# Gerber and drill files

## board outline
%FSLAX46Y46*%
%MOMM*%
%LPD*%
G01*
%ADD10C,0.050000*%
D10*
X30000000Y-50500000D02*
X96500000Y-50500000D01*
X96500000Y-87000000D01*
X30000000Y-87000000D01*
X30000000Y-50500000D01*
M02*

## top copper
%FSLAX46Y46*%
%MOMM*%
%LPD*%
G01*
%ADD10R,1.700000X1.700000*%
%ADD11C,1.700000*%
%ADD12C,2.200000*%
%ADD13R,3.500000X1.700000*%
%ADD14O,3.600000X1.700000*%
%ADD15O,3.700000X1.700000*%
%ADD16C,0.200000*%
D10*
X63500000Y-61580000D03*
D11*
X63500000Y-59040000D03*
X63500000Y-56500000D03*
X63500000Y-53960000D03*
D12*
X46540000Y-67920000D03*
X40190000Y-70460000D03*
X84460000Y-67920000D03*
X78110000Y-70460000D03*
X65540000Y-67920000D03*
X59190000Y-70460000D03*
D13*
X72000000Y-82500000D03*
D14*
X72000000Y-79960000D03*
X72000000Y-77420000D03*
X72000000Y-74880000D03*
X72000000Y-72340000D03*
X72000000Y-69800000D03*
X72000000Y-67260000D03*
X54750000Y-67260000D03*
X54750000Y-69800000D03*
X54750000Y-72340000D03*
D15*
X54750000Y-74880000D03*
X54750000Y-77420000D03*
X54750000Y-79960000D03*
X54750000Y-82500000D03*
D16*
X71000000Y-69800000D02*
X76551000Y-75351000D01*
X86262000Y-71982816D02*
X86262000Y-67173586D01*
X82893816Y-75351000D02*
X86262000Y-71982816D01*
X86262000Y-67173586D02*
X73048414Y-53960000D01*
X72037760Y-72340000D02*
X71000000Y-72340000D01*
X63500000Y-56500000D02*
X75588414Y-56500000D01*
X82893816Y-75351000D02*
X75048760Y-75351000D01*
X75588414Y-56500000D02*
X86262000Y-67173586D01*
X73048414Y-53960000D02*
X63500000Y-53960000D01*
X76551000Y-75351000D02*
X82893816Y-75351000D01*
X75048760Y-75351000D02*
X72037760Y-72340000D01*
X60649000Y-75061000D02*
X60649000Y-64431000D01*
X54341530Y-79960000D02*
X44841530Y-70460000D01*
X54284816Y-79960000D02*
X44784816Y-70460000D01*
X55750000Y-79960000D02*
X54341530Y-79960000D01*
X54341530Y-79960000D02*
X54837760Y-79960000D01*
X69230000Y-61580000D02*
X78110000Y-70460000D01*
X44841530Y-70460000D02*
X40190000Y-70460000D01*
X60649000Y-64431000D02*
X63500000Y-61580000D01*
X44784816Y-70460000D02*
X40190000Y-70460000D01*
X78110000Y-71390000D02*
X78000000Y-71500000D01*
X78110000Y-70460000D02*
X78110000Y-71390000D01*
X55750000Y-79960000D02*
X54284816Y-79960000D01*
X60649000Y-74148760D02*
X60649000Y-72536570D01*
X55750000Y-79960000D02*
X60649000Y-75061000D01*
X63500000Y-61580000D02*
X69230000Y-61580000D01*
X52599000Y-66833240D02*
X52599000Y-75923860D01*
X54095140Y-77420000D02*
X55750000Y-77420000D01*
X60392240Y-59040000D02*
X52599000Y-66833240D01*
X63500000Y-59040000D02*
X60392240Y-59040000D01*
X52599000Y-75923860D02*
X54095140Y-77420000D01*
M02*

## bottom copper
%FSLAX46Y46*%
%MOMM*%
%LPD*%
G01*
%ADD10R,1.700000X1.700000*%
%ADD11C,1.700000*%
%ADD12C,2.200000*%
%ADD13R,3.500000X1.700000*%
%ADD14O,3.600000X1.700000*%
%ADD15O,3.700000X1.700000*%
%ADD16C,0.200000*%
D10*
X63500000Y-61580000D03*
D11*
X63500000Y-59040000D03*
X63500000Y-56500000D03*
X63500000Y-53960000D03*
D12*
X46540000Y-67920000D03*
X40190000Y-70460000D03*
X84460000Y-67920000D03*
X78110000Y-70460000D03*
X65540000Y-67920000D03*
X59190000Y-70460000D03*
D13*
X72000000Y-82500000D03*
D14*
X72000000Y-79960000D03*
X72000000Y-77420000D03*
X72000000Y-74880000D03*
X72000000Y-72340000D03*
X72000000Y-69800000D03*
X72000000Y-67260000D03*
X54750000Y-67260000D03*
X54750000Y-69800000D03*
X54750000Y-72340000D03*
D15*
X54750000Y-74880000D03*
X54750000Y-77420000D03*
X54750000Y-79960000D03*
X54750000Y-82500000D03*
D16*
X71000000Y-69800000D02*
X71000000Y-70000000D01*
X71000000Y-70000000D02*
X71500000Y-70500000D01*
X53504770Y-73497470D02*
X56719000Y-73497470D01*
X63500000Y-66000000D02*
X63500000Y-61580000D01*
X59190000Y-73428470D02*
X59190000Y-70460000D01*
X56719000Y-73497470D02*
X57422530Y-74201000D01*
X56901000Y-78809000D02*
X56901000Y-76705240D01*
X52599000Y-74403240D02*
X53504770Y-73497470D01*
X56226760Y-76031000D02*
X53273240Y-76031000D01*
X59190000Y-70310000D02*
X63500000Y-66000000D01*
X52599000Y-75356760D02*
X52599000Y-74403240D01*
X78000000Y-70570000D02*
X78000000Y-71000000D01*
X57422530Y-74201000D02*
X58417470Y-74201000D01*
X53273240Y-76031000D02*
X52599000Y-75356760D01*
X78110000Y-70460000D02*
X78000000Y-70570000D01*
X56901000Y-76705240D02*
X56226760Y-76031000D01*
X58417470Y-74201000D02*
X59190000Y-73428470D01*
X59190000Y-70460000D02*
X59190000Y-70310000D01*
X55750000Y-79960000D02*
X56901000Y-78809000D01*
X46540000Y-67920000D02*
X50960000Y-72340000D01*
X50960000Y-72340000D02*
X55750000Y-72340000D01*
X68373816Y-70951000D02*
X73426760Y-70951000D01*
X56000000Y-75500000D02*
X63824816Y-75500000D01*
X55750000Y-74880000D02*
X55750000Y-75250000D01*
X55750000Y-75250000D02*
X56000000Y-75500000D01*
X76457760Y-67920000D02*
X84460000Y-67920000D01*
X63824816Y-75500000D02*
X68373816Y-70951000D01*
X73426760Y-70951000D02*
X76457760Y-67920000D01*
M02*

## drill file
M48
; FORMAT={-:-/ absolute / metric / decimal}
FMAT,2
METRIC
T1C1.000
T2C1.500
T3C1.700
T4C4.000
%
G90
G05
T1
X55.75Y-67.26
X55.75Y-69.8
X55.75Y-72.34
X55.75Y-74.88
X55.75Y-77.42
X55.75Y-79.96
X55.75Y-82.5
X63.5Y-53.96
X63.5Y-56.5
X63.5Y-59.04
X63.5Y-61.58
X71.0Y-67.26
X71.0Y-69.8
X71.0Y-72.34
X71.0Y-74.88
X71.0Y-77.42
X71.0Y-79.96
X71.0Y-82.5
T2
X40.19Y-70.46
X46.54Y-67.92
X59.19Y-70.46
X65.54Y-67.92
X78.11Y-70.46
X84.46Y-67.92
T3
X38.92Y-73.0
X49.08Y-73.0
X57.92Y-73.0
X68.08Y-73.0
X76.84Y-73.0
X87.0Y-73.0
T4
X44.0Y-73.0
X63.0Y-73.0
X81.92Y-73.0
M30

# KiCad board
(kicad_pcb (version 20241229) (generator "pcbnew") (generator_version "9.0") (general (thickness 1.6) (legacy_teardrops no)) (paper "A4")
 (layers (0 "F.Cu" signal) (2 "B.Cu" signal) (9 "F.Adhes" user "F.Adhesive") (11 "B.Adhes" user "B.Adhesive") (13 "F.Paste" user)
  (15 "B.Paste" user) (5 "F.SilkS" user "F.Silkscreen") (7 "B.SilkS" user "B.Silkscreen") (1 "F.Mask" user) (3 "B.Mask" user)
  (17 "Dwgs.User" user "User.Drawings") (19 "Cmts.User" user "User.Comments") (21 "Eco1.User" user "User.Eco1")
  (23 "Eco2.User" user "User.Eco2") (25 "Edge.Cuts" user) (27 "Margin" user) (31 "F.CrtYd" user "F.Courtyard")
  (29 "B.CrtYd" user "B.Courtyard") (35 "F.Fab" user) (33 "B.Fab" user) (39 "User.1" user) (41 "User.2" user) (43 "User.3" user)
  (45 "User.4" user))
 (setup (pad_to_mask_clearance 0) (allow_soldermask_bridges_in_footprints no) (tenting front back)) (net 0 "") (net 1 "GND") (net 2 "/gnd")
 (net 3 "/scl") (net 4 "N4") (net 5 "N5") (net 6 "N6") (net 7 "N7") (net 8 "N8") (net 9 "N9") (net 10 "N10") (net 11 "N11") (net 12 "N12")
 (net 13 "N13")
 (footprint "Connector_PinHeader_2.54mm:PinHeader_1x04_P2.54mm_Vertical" (layer "F.Cu") (at 63.5 61.58 180)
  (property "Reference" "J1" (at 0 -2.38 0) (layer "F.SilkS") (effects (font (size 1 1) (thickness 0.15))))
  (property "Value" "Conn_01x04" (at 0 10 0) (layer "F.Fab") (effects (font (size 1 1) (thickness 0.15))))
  (pad "1" thru_hole rect (at 0 0 180) (size 1.7 1.7) (drill 1) (layers "*.Cu" "*.Mask") (remove_unused_layers no) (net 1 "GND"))
  (pad "2" thru_hole circle (at 0 2.54 180) (size 1.7 1.7) (drill 1) (layers "*.Cu" "*.Mask") (remove_unused_layers no) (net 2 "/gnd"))
  (pad "3" thru_hole circle (at 0 5.08 180) (size 1.7 1.7) (drill 1) (layers "*.Cu" "*.Mask") (remove_unused_layers no) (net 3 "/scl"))
  (pad "4" thru_hole circle (at 0 7.62 180) (size 1.7 1.7) (drill 1) (layers "*.Cu" "*.Mask") (remove_unused_layers no) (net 3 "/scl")))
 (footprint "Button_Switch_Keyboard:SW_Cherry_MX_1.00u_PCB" (layer "F.Cu") (at 46.54 67.92)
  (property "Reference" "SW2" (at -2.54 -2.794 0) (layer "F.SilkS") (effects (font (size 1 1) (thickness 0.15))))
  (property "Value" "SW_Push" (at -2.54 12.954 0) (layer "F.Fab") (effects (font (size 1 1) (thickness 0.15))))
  (pad "" np_thru_hole circle (at -7.62 5.08) (size 1.7 1.7) (drill 1.7) (layers "*.Cu" "*.Mask"))
  (pad "" np_thru_hole circle (at -2.54 5.08) (size 4 4) (drill 4) (layers "*.Cu" "*.Mask"))
  (pad "" np_thru_hole circle (at 2.54 5.08) (size 1.7 1.7) (drill 1.7) (layers "*.Cu" "*.Mask"))
  (pad "1" thru_hole circle (at 0 0) (size 2.2 2.2) (drill 1.5) (layers "*.Cu" "*.Mask") (remove_unused_layers no) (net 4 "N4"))
  (pad "2" thru_hole circle (at -6.35 2.54) (size 2.2 2.2) (drill 1.5) (layers "*.Cu" "*.Mask") (remove_unused_layers no) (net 1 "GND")))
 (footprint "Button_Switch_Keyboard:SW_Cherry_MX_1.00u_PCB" (layer "F.Cu") (at 84.46 67.92)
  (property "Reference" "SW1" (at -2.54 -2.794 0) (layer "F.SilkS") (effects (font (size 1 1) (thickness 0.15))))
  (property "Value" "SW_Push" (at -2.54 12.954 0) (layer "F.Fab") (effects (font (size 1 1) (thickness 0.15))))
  (pad "" np_thru_hole circle (at -7.62 5.08) (size 1.7 1.7) (drill 1.7) (layers "*.Cu" "*.Mask"))
  (pad "" np_thru_hole circle (at -2.54 5.08) (size 4 4) (drill 4) (layers "*.Cu" "*.Mask"))
  (pad "" np_thru_hole circle (at 2.54 5.08) (size 1.7 1.7) (drill 1.7) (layers "*.Cu" "*.Mask"))
  (pad "1" thru_hole circle (at 0 0) (size 2.2 2.2) (drill 1.5) (layers "*.Cu" "*.Mask") (remove_unused_layers no) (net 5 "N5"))
  (pad "2" thru_hole circle (at -6.35 2.54) (size 2.2 2.2) (drill 1.5) (layers "*.Cu" "*.Mask") (remove_unused_layers no) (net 1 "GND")))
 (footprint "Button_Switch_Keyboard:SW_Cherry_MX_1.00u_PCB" (layer "F.Cu") (at 65.54 67.92)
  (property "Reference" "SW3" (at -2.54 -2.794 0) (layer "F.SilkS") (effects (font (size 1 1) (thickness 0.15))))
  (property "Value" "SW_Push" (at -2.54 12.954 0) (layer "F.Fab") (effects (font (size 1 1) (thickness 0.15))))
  (pad "" np_thru_hole circle (at -7.62 5.08) (size 1.7 1.7) (drill 1.7) (layers "*.Cu" "*.Mask"))
  (pad "" np_thru_hole circle (at -2.54 5.08) (size 4 4) (drill 4) (layers "*.Cu" "*.Mask"))
  (pad "" np_thru_hole circle (at 2.54 5.08) (size 1.7 1.7) (drill 1.7) (layers "*.Cu" "*.Mask"))
  (pad "1" thru_hole circle (at 0 0) (size 2.2 2.2) (drill 1.5) (layers "*.Cu" "*.Mask") (remove_unused_layers no) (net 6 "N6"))
  (pad "2" thru_hole circle (at -6.35 2.54) (size 2.2 2.2) (drill 1.5) (layers "*.Cu" "*.Mask") (remove_unused_layers no) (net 1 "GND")))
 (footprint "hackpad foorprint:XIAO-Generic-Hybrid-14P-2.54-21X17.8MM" (layer "F.Cu") (at 63.375 74.88 180)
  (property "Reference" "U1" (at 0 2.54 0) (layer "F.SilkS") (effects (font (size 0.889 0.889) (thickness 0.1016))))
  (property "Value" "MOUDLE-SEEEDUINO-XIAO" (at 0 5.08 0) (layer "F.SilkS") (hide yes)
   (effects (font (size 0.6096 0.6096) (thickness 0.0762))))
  (pad "1" thru_hole rect (at -7.625 -7.62 180) (size 3.5 1.7) (drill 1 (offset -1 0)) (layers "*.Cu" "*.Mask") (remove_unused_layers no)
   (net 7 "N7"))
  (pad "2" thru_hole oval (at -7.625 -5.08 180) (size 3.6 1.7) (drill 1 (offset -1 0)) (layers "*.Cu" "*.Mask") (remove_unused_layers no)
   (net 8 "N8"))
  (pad "3" thru_hole oval (at -7.625 -2.54 180) (size 3.6 1.7) (drill 1 (offset -1 0)) (layers "*.Cu" "*.Mask") (remove_unused_layers no)
   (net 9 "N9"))
  (pad "4" thru_hole oval (at -7.625 0 180) (size 3.6 1.7) (drill 1 (offset -1 0)) (layers "*.Cu" "*.Mask") (remove_unused_layers no)
   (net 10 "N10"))
  (pad "5" thru_hole oval (at -7.625 2.54 180) (size 3.6 1.7) (drill 1 (offset -1 0)) (layers "*.Cu" "*.Mask") (remove_unused_layers no)
   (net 3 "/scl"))
  (pad "6" thru_hole oval (at -7.625 5.08) (size 3.6 1.7) (drill 1 (offset 1 0)) (layers "*.Cu" "*.Mask") (remove_unused_layers no)
   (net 3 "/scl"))
  (pad "7" thru_hole oval (at -7.625 7.62 180) (size 3.6 1.7) (drill 1 (offset -1 0)) (layers "*.Cu" "*.Mask") (remove_unused_layers no)
   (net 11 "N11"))
  (pad "8" thru_hole oval (at 7.625 7.62 180) (size 3.6 1.7) (drill 1 (offset 1 0)) (layers "*.Cu" "*.Mask") (remove_unused_layers no)
   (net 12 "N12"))
  (pad "9" thru_hole oval (at 7.625 5.08 180) (size 3.6 1.7) (drill 1 (offset 1 0)) (layers "*.Cu" "*.Mask") (remove_unused_layers no)
   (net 6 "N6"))
  (pad "10" thru_hole oval (at 7.625 2.54 180) (size 3.6 1.7) (drill 1 (offset 1 0)) (layers "*.Cu" "*.Mask") (remove_unused_layers no)
   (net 4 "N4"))
  (pad "11" thru_hole oval (at 7.625 0 180) (size 3.7 1.7) (drill 1 (offset 1 0)) (layers "*.Cu" "*.Mask") (remove_unused_layers no)
   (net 5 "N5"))
  (pad "12" thru_hole oval (at 7.625 -2.54 180) (size 3.7 1.7) (drill 1 (offset 1 0)) (layers "*.Cu" "*.Mask") (remove_unused_layers no)
   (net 2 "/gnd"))
  (pad "13" thru_hole oval (at 7.625 -5.08 180) (size 3.7 1.7) (drill 1 (offset 1 0)) (layers "*.Cu" "*.Mask") (remove_unused_layers no)
   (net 1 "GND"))
  (pad "14" thru_hole oval (at 7.625 -7.62 180) (size 3.7 1.7) (drill 1 (offset 1 0)) (layers "*.Cu" "*.Mask") (remove_unused_layers no)
   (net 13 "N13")))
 (gr_rect (start 30 50.5) (end 96.5 87) (stroke (width 0.05) (type default)) (fill no) (layer "Edge.Cuts"))
 (segment (start 71 69.8) (end 76.551 75.351) (width 0.2) (layer "F.Cu") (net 3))
 (segment (start 86.262 71.982816) (end 86.262 67.173586) (width 0.2) (layer "F.Cu") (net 3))
 (segment (start 82.893816 75.351) (end 86.262 71.982816) (width 0.2) (layer "F.Cu") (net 3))
 (segment (start 86.262 67.173586) (end 73.048414 53.96) (width 0.2) (layer "F.Cu") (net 3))
 (segment (start 72.03776 72.34) (end 71 72.34) (width 0.2) (layer "F.Cu") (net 3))
 (segment (start 63.5 56.5) (end 75.588414 56.5) (width 0.2) (layer "F.Cu") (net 3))
 (segment (start 82.893816 75.351) (end 75.04876 75.351) (width 0.2) (layer "F.Cu") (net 3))
 (segment (start 75.588414 56.5) (end 86.262 67.173586) (width 0.2) (layer "F.Cu") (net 3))
 (segment (start 73.048414 53.96) (end 63.5 53.96) (width 0.2) (layer "F.Cu") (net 3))
 (segment (start 76.551 75.351) (end 82.893816 75.351) (width 0.2) (layer "F.Cu") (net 3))
 (segment (start 75.04876 75.351) (end 72.03776 72.34) (width 0.2) (layer "F.Cu") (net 3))
 (segment (start 71 69.8) (end 71 70) (width 0.2) (layer "B.Cu") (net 3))
 (segment (start 71 70) (end 71.5 70.5) (width 0.2) (layer "B.Cu") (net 3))
 (segment (start 60.649 75.061) (end 60.649 64.431) (width 0.2) (layer "F.Cu") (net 1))
 (segment (start 54.34153 79.96) (end 44.84153 70.46) (width 0.2) (layer "F.Cu") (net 1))
 (segment (start 54.284816 79.96) (end 44.784816 70.46) (width 0.2) (layer "F.Cu") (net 1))
 (segment (start 55.75 79.96) (end 54.34153 79.96) (width 0.2) (layer "F.Cu") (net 1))
 (segment (start 54.34153 79.96) (end 54.83776 79.96) (width 0.2) (layer "F.Cu") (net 1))
 (segment (start 69.23 61.58) (end 78.11 70.46) (width 0.2) (layer "F.Cu") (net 1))
 (segment (start 44.84153 70.46) (end 40.19 70.46) (width 0.2) (layer "F.Cu") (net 1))
 (segment (start 60.649 64.431) (end 63.5 61.58) (width 0.2) (layer "F.Cu") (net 1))
 (segment (start 44.784816 70.46) (end 40.19 70.46) (width 0.2) (layer "F.Cu") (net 1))
 (segment (start 78.11 71.39) (end 78 71.5) (width 0.2) (layer "F.Cu") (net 1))
 (segment (start 78.11 70.46) (end 78.11 71.39) (width 0.2) (layer "F.Cu") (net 1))
 (segment (start 55.75 79.96) (end 54.284816 79.96) (width 0.2) (layer "F.Cu") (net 1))
 (segment (start 60.649 74.14876) (end 60.649 72.53657) (width 0.2) (layer "F.Cu") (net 1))
 (segment (start 55.75 79.96) (end 60.649 75.061) (width 0.2) (layer "F.Cu") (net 1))
 (segment (start 63.5 61.58) (end 69.23 61.58) (width 0.2) (layer "F.Cu") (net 1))
 (segment (start 53.50477 73.49747) (end 56.719 73.49747) (width 0.2) (layer "B.Cu") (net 1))
 (segment (start 63.5 66) (end 63.5 61.58) (width 0.2) (layer "B.Cu") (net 1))
 (segment (start 59.19 73.42847) (end 59.19 70.46) (width 0.2) (layer "B.Cu") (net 1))
 (segment (start 56.719 73.49747) (end 57.42253 74.201) (width 0.2) (layer "B.Cu") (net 1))
 (segment (start 56.901 78.809) (end 56.901 76.70524) (width 0.2) (layer "B.Cu") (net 1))
 (segment (start 52.599 74.40324) (end 53.50477 73.49747) (width 0.2) (layer "B.Cu") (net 1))
 (segment (start 56.22676 76.031) (end 53.27324 76.031) (width 0.2) (layer "B.Cu") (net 1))
 (segment (start 59.19 70.31) (end 63.5 66) (width 0.2) (layer "B.Cu") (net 1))
 (segment (start 52.599 75.35676) (end 52.599 74.40324) (width 0.2) (layer "B.Cu") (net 1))
 (segment (start 78 70.57) (end 78 71) (width 0.2) (layer "B.Cu") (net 1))
 (segment (start 57.42253 74.201) (end 58.41747 74.201) (width 0.2) (layer "B.Cu") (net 1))
 (segment (start 53.27324 76.031) (end 52.599 75.35676) (width 0.2) (layer "B.Cu") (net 1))
 (segment (start 78.11 70.46) (end 78 70.57) (width 0.2) (layer "B.Cu") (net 1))
 (segment (start 56.901 76.70524) (end 56.22676 76.031) (width 0.2) (layer "B.Cu") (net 1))
 (segment (start 58.41747 74.201) (end 59.19 73.42847) (width 0.2) (layer "B.Cu") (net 1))
 (segment (start 59.19 70.46) (end 59.19 70.31) (width 0.2) (layer "B.Cu") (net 1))
 (segment (start 55.75 79.96) (end 56.901 78.809) (width 0.2) (layer "B.Cu") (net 1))
 (segment (start 46.54 67.92) (end 50.96 72.34) (width 0.2) (layer "B.Cu") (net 4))
 (segment (start 50.96 72.34) (end 55.75 72.34) (width 0.2) (layer "B.Cu") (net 4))
 (segment (start 68.373816 70.951) (end 73.42676 70.951) (width 0.2) (layer "B.Cu") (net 5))
 (segment (start 56 75.5) (end 63.824816 75.5) (width 0.2) (layer "B.Cu") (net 5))
 (segment (start 55.75 74.88) (end 55.75 75.25) (width 0.2) (layer "B.Cu") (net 5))
 (segment (start 55.75 75.25) (end 56 75.5) (width 0.2) (layer "B.Cu") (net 5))
 (segment (start 76.45776 67.92) (end 84.46 67.92) (width 0.2) (layer "B.Cu") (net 5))
 (segment (start 63.824816 75.5) (end 68.373816 70.951) (width 0.2) (layer "B.Cu") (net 5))
 (segment (start 73.42676 70.951) (end 76.45776 67.92) (width 0.2) (layer "B.Cu") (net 5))
 (segment (start 52.599 66.83324) (end 52.599 75.92386) (width 0.2) (layer "F.Cu") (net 2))
 (segment (start 54.09514 77.42) (end 55.75 77.42) (width 0.2) (layer "F.Cu") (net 2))
 (segment (start 60.39224 59.04) (end 52.599 66.83324) (width 0.2) (layer "F.Cu") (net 2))
 (segment (start 63.5 59.04) (end 60.39224 59.04) (width 0.2) (layer "F.Cu") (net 2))
 (segment (start 52.599 75.92386) (end 54.09514 77.42) (width 0.2) (layer "F.Cu") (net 2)))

